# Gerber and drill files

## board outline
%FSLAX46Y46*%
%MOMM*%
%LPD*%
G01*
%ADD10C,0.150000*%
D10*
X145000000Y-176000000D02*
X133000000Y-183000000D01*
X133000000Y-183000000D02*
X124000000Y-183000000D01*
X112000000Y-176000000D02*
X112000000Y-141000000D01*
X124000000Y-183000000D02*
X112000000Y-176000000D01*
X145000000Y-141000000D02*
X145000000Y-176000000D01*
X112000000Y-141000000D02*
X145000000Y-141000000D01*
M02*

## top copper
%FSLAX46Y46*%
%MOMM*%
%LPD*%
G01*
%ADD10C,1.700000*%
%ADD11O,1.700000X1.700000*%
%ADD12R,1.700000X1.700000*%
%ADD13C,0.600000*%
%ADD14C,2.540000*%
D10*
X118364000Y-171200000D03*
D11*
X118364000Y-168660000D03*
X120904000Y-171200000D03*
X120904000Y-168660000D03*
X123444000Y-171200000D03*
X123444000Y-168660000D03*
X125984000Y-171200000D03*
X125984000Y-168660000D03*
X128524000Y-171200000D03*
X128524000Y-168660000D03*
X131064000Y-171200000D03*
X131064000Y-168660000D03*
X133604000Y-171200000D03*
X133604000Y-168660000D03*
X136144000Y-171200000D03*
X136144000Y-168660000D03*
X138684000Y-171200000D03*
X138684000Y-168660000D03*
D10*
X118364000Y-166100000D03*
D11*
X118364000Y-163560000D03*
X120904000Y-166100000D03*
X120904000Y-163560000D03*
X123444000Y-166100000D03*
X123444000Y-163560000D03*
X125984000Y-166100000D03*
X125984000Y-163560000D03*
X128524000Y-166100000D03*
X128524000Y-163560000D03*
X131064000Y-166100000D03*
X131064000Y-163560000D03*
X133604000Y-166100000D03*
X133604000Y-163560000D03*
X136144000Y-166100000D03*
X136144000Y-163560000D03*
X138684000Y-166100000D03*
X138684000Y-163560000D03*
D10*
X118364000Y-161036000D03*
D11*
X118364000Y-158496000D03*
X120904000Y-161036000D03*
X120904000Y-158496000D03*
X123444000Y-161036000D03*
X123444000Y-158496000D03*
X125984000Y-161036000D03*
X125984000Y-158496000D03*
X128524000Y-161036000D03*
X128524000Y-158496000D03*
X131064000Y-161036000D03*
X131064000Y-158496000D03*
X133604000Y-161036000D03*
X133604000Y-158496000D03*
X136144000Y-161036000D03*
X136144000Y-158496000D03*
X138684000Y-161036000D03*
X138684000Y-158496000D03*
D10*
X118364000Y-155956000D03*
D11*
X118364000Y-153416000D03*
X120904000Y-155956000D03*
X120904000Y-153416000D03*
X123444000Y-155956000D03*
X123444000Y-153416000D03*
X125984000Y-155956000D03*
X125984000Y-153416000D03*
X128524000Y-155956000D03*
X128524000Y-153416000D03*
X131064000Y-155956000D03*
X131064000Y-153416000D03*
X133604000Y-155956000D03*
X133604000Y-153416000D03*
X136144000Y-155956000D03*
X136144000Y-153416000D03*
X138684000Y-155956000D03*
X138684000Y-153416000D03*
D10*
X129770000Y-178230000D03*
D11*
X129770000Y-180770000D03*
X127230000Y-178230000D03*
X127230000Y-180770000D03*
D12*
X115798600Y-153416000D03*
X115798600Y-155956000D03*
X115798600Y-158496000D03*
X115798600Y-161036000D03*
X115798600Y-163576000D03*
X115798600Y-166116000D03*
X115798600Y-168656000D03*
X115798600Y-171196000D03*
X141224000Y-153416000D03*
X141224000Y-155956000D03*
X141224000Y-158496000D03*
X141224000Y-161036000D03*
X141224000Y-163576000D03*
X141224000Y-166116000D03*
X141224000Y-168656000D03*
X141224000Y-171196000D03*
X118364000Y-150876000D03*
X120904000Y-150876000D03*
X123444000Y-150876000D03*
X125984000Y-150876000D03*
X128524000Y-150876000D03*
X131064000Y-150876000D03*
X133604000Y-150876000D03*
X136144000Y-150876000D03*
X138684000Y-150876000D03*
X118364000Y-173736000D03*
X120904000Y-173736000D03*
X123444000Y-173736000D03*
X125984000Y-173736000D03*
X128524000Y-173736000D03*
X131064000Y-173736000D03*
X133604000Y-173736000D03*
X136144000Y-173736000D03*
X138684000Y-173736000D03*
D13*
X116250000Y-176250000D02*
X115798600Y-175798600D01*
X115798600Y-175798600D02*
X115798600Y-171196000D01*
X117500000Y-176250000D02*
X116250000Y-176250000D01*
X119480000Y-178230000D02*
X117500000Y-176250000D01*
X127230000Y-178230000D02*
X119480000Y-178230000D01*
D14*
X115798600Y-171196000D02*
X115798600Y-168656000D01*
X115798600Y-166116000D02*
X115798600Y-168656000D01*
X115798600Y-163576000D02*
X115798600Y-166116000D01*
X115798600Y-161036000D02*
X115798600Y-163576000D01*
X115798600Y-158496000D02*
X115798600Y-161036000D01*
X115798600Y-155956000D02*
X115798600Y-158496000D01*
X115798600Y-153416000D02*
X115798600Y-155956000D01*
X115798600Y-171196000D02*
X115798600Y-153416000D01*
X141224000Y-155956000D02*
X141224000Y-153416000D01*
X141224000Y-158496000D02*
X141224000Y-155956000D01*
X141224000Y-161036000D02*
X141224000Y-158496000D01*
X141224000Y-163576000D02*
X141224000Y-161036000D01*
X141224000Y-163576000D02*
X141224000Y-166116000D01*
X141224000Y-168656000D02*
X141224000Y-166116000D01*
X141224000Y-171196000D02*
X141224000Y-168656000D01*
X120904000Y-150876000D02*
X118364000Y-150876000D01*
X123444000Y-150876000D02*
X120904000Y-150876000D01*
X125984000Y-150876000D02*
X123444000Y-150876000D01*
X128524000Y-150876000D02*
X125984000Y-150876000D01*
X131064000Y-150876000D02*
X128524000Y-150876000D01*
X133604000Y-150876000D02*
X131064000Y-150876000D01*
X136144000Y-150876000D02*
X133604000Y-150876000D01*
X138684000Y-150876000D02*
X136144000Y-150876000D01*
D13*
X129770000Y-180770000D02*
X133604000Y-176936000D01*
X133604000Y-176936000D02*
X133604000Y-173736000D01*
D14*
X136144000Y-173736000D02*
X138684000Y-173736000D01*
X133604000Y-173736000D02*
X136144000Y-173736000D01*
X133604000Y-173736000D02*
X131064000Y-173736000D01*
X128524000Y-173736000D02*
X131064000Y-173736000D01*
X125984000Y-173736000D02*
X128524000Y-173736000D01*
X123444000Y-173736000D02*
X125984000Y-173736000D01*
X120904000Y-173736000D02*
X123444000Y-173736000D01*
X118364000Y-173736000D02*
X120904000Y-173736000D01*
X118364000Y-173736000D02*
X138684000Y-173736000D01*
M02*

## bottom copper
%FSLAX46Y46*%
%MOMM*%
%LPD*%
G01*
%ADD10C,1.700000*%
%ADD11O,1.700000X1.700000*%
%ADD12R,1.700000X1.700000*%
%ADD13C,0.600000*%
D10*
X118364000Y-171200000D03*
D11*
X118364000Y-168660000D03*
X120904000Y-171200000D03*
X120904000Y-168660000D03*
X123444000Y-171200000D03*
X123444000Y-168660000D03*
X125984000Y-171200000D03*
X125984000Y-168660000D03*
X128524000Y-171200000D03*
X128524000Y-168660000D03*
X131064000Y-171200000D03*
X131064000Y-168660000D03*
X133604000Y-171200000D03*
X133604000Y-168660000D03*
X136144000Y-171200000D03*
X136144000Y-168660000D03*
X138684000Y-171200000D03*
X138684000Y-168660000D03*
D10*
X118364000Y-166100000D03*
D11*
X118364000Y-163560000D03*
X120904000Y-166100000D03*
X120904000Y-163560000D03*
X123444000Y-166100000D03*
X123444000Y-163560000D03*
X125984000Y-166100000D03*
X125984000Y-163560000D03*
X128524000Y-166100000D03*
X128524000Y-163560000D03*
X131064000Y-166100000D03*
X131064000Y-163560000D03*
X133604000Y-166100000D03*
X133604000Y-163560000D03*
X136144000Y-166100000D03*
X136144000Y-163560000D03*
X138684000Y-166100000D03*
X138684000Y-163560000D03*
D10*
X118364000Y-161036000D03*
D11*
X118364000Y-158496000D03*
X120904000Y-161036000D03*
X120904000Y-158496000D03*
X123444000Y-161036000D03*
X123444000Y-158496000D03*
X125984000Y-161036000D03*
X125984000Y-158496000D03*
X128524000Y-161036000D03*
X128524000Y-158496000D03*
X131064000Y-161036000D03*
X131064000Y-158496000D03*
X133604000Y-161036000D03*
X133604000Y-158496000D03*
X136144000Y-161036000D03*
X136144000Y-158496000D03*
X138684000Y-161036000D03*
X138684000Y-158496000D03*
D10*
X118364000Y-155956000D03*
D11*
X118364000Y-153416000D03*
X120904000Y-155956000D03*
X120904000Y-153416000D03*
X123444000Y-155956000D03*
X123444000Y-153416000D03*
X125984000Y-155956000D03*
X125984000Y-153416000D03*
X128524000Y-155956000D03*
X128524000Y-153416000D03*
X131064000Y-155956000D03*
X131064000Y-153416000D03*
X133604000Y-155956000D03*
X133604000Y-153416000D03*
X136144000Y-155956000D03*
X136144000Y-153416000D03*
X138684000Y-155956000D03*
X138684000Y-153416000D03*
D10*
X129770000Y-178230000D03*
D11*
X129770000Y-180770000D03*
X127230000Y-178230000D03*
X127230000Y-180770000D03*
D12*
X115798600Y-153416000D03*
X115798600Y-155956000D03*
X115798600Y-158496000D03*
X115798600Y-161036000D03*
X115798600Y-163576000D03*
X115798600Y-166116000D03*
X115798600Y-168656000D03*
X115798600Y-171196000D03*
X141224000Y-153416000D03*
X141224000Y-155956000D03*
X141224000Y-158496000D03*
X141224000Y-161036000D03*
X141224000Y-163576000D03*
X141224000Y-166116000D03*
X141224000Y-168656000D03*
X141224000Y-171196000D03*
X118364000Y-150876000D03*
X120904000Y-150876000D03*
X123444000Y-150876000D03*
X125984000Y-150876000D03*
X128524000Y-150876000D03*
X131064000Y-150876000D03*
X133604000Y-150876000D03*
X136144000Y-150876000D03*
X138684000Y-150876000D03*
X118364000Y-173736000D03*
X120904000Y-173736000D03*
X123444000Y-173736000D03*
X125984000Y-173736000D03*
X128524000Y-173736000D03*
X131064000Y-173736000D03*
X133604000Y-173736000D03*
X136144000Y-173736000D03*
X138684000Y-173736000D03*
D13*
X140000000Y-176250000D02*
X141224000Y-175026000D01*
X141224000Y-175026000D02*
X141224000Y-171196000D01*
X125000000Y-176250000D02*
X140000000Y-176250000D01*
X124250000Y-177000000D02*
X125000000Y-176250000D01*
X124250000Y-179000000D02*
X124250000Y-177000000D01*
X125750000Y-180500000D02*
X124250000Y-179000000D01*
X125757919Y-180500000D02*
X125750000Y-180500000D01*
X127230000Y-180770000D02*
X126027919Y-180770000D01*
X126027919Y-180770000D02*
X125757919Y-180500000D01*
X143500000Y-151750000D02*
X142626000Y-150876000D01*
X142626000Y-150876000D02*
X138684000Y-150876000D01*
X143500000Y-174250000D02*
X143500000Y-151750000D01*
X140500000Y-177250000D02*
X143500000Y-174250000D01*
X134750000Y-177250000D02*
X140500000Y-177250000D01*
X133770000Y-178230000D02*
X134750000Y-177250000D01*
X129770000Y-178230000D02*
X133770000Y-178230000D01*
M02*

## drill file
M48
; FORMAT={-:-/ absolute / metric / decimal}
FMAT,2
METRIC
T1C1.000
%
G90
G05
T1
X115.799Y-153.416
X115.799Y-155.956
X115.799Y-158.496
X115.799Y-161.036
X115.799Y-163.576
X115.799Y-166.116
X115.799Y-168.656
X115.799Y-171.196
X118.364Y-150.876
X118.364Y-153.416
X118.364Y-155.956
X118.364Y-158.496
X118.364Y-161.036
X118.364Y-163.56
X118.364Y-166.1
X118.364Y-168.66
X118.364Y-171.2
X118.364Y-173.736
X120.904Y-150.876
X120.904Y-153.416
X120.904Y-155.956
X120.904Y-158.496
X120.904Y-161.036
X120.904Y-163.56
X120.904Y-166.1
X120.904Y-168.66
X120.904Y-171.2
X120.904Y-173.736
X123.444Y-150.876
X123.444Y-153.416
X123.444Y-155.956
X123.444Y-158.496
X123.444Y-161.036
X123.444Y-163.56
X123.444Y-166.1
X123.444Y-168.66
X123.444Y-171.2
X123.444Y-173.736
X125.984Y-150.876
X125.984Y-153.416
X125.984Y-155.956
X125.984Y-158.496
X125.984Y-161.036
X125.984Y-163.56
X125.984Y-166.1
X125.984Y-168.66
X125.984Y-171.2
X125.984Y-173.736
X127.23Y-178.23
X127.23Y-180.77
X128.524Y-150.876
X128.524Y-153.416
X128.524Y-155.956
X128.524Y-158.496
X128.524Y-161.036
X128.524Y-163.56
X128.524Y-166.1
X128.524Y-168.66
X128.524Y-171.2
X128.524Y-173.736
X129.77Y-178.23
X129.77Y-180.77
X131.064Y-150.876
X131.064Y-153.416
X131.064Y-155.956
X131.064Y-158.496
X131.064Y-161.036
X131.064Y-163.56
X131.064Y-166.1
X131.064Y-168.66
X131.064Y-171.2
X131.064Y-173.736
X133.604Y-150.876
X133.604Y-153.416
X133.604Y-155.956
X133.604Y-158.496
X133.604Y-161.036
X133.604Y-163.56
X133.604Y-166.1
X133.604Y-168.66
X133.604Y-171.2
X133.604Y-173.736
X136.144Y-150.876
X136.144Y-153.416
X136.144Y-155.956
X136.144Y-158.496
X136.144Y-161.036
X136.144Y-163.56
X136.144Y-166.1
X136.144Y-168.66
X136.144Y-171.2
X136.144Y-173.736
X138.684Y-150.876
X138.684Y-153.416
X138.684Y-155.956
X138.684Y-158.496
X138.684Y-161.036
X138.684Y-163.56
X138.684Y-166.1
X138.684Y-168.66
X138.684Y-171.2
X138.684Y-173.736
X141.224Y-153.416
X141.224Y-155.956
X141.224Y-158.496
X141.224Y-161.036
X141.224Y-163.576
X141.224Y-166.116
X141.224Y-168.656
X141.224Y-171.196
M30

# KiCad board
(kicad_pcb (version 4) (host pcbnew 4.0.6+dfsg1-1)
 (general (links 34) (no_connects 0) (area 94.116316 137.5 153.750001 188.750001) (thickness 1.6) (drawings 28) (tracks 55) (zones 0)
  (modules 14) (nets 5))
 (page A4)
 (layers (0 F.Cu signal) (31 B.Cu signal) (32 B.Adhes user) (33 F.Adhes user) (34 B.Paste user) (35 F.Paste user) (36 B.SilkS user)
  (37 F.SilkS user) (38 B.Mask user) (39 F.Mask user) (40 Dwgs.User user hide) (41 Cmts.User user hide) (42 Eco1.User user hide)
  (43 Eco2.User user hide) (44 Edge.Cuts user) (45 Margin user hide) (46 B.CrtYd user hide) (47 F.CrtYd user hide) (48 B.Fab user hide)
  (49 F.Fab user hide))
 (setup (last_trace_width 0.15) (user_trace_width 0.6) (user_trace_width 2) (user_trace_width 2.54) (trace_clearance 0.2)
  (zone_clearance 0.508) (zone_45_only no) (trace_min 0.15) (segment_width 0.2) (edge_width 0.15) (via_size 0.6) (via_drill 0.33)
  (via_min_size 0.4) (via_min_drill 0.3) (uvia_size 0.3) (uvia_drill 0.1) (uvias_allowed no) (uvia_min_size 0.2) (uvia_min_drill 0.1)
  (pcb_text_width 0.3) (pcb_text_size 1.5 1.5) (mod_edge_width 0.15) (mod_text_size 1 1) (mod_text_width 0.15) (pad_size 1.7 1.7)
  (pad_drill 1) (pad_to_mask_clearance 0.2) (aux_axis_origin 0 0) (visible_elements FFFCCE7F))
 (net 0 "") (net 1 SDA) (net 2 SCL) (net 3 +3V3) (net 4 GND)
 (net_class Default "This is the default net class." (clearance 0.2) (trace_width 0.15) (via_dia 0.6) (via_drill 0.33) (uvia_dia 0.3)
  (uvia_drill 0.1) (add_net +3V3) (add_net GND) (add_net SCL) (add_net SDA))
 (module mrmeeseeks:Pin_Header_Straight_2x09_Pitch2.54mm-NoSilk (layer F.Cu) (at 118.364 171.2 90)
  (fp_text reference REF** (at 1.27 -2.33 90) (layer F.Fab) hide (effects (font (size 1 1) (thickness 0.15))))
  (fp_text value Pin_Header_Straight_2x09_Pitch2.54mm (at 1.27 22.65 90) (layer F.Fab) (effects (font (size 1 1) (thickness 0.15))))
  (pad 1 thru_hole circle (at 0 0 90) (size 1.7 1.7) (drill 1) (layers *.Cu *.Mask))
  (pad 2 thru_hole oval (at 2.54 0 90) (size 1.7 1.7) (drill 1) (layers *.Cu *.Mask))
  (pad 3 thru_hole oval (at 0 2.54 90) (size 1.7 1.7) (drill 1) (layers *.Cu *.Mask))
  (pad 4 thru_hole oval (at 2.54 2.54 90) (size 1.7 1.7) (drill 1) (layers *.Cu *.Mask))
  (pad 5 thru_hole oval (at 0 5.08 90) (size 1.7 1.7) (drill 1) (layers *.Cu *.Mask))
  (pad 6 thru_hole oval (at 2.54 5.08 90) (size 1.7 1.7) (drill 1) (layers *.Cu *.Mask))
  (pad 7 thru_hole oval (at 0 7.62 90) (size 1.7 1.7) (drill 1) (layers *.Cu *.Mask))
  (pad 8 thru_hole oval (at 2.54 7.62 90) (size 1.7 1.7) (drill 1) (layers *.Cu *.Mask))
  (pad 9 thru_hole oval (at 0 10.16 90) (size 1.7 1.7) (drill 1) (layers *.Cu *.Mask))
  (pad 10 thru_hole oval (at 2.54 10.16 90) (size 1.7 1.7) (drill 1) (layers *.Cu *.Mask))
  (pad 11 thru_hole oval (at 0 12.7 90) (size 1.7 1.7) (drill 1) (layers *.Cu *.Mask))
  (pad 12 thru_hole oval (at 2.54 12.7 90) (size 1.7 1.7) (drill 1) (layers *.Cu *.Mask))
  (pad 13 thru_hole oval (at 0 15.24 90) (size 1.7 1.7) (drill 1) (layers *.Cu *.Mask))
  (pad 14 thru_hole oval (at 2.54 15.24 90) (size 1.7 1.7) (drill 1) (layers *.Cu *.Mask))
  (pad 15 thru_hole oval (at 0 17.78 90) (size 1.7 1.7) (drill 1) (layers *.Cu *.Mask))
  (pad 16 thru_hole oval (at 2.54 17.78 90) (size 1.7 1.7) (drill 1) (layers *.Cu *.Mask))
  (pad 17 thru_hole oval (at 0 20.32 90) (size 1.7 1.7) (drill 1) (layers *.Cu *.Mask))
  (pad 18 thru_hole oval (at 2.54 20.32 90) (size 1.7 1.7) (drill 1) (layers *.Cu *.Mask)))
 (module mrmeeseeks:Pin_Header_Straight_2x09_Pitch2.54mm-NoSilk (layer F.Cu) (at 118.364 166.1 90)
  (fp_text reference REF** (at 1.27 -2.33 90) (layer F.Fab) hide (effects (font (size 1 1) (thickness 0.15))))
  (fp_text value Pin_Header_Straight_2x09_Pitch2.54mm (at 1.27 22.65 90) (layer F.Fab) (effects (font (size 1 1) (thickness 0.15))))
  (pad 1 thru_hole circle (at 0 0 90) (size 1.7 1.7) (drill 1) (layers *.Cu *.Mask))
  (pad 2 thru_hole oval (at 2.54 0 90) (size 1.7 1.7) (drill 1) (layers *.Cu *.Mask))
  (pad 3 thru_hole oval (at 0 2.54 90) (size 1.7 1.7) (drill 1) (layers *.Cu *.Mask))
  (pad 4 thru_hole oval (at 2.54 2.54 90) (size 1.7 1.7) (drill 1) (layers *.Cu *.Mask))
  (pad 5 thru_hole oval (at 0 5.08 90) (size 1.7 1.7) (drill 1) (layers *.Cu *.Mask))
  (pad 6 thru_hole oval (at 2.54 5.08 90) (size 1.7 1.7) (drill 1) (layers *.Cu *.Mask))
  (pad 7 thru_hole oval (at 0 7.62 90) (size 1.7 1.7) (drill 1) (layers *.Cu *.Mask))
  (pad 8 thru_hole oval (at 2.54 7.62 90) (size 1.7 1.7) (drill 1) (layers *.Cu *.Mask))
  (pad 9 thru_hole oval (at 0 10.16 90) (size 1.7 1.7) (drill 1) (layers *.Cu *.Mask))
  (pad 10 thru_hole oval (at 2.54 10.16 90) (size 1.7 1.7) (drill 1) (layers *.Cu *.Mask))
  (pad 11 thru_hole oval (at 0 12.7 90) (size 1.7 1.7) (drill 1) (layers *.Cu *.Mask))
  (pad 12 thru_hole oval (at 2.54 12.7 90) (size 1.7 1.7) (drill 1) (layers *.Cu *.Mask))
  (pad 13 thru_hole oval (at 0 15.24 90) (size 1.7 1.7) (drill 1) (layers *.Cu *.Mask))
  (pad 14 thru_hole oval (at 2.54 15.24 90) (size 1.7 1.7) (drill 1) (layers *.Cu *.Mask))
  (pad 15 thru_hole oval (at 0 17.78 90) (size 1.7 1.7) (drill 1) (layers *.Cu *.Mask))
  (pad 16 thru_hole oval (at 2.54 17.78 90) (size 1.7 1.7) (drill 1) (layers *.Cu *.Mask))
  (pad 17 thru_hole oval (at 0 20.32 90) (size 1.7 1.7) (drill 1) (layers *.Cu *.Mask))
  (pad 18 thru_hole oval (at 2.54 20.32 90) (size 1.7 1.7) (drill 1) (layers *.Cu *.Mask)))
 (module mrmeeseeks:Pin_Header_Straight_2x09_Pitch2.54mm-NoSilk (layer F.Cu) (at 118.364 161.036 90)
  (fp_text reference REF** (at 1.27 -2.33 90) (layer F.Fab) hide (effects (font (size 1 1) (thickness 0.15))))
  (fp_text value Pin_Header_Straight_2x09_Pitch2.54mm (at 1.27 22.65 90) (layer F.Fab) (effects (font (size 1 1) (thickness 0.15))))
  (pad 1 thru_hole circle (at 0 0 90) (size 1.7 1.7) (drill 1) (layers *.Cu *.Mask))
  (pad 2 thru_hole oval (at 2.54 0 90) (size 1.7 1.7) (drill 1) (layers *.Cu *.Mask))
  (pad 3 thru_hole oval (at 0 2.54 90) (size 1.7 1.7) (drill 1) (layers *.Cu *.Mask))
  (pad 4 thru_hole oval (at 2.54 2.54 90) (size 1.7 1.7) (drill 1) (layers *.Cu *.Mask))
  (pad 5 thru_hole oval (at 0 5.08 90) (size 1.7 1.7) (drill 1) (layers *.Cu *.Mask))
  (pad 6 thru_hole oval (at 2.54 5.08 90) (size 1.7 1.7) (drill 1) (layers *.Cu *.Mask))
  (pad 7 thru_hole oval (at 0 7.62 90) (size 1.7 1.7) (drill 1) (layers *.Cu *.Mask))
  (pad 8 thru_hole oval (at 2.54 7.62 90) (size 1.7 1.7) (drill 1) (layers *.Cu *.Mask))
  (pad 9 thru_hole oval (at 0 10.16 90) (size 1.7 1.7) (drill 1) (layers *.Cu *.Mask))
  (pad 10 thru_hole oval (at 2.54 10.16 90) (size 1.7 1.7) (drill 1) (layers *.Cu *.Mask))
  (pad 11 thru_hole oval (at 0 12.7 90) (size 1.7 1.7) (drill 1) (layers *.Cu *.Mask))
  (pad 12 thru_hole oval (at 2.54 12.7 90) (size 1.7 1.7) (drill 1) (layers *.Cu *.Mask))
  (pad 13 thru_hole oval (at 0 15.24 90) (size 1.7 1.7) (drill 1) (layers *.Cu *.Mask))
  (pad 14 thru_hole oval (at 2.54 15.24 90) (size 1.7 1.7) (drill 1) (layers *.Cu *.Mask))
  (pad 15 thru_hole oval (at 0 17.78 90) (size 1.7 1.7) (drill 1) (layers *.Cu *.Mask))
  (pad 16 thru_hole oval (at 2.54 17.78 90) (size 1.7 1.7) (drill 1) (layers *.Cu *.Mask))
  (pad 17 thru_hole oval (at 0 20.32 90) (size 1.7 1.7) (drill 1) (layers *.Cu *.Mask))
  (pad 18 thru_hole oval (at 2.54 20.32 90) (size 1.7 1.7) (drill 1) (layers *.Cu *.Mask)))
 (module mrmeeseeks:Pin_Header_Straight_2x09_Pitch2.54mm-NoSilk (layer F.Cu) (at 118.364 155.956 90)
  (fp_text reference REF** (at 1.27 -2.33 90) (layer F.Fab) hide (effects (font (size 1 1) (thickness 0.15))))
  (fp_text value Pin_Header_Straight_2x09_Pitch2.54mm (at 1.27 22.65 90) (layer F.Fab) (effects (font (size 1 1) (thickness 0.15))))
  (pad 1 thru_hole circle (at 0 0 90) (size 1.7 1.7) (drill 1) (layers *.Cu *.Mask))
  (pad 2 thru_hole oval (at 2.54 0 90) (size 1.7 1.7) (drill 1) (layers *.Cu *.Mask))
  (pad 3 thru_hole oval (at 0 2.54 90) (size 1.7 1.7) (drill 1) (layers *.Cu *.Mask))
  (pad 4 thru_hole oval (at 2.54 2.54 90) (size 1.7 1.7) (drill 1) (layers *.Cu *.Mask))
  (pad 5 thru_hole oval (at 0 5.08 90) (size 1.7 1.7) (drill 1) (layers *.Cu *.Mask))
  (pad 6 thru_hole oval (at 2.54 5.08 90) (size 1.7 1.7) (drill 1) (layers *.Cu *.Mask))
  (pad 7 thru_hole oval (at 0 7.62 90) (size 1.7 1.7) (drill 1) (layers *.Cu *.Mask))
  (pad 8 thru_hole oval (at 2.54 7.62 90) (size 1.7 1.7) (drill 1) (layers *.Cu *.Mask))
  (pad 9 thru_hole oval (at 0 10.16 90) (size 1.7 1.7) (drill 1) (layers *.Cu *.Mask))
  (pad 10 thru_hole oval (at 2.54 10.16 90) (size 1.7 1.7) (drill 1) (layers *.Cu *.Mask))
  (pad 11 thru_hole oval (at 0 12.7 90) (size 1.7 1.7) (drill 1) (layers *.Cu *.Mask))
  (pad 12 thru_hole oval (at 2.54 12.7 90) (size 1.7 1.7) (drill 1) (layers *.Cu *.Mask))
  (pad 13 thru_hole oval (at 0 15.24 90) (size 1.7 1.7) (drill 1) (layers *.Cu *.Mask))
  (pad 14 thru_hole oval (at 2.54 15.24 90) (size 1.7 1.7) (drill 1) (layers *.Cu *.Mask))
  (pad 15 thru_hole oval (at 0 17.78 90) (size 1.7 1.7) (drill 1) (layers *.Cu *.Mask))
  (pad 16 thru_hole oval (at 2.54 17.78 90) (size 1.7 1.7) (drill 1) (layers *.Cu *.Mask))
  (pad 17 thru_hole oval (at 0 20.32 90) (size 1.7 1.7) (drill 1) (layers *.Cu *.Mask))
  (pad 18 thru_hole oval (at 2.54 20.32 90) (size 1.7 1.7) (drill 1) (layers *.Cu *.Mask)))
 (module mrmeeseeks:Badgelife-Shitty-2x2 (layer F.Cu) (at 128.5 179.5)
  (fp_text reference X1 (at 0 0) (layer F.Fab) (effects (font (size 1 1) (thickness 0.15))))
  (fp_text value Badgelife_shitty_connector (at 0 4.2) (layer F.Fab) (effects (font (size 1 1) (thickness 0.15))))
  (pad 4 thru_hole circle (at 1.27 -1.27) (size 1.7 1.7) (drill 1) (layers *.Cu *.Mask) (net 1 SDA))
  (pad 3 thru_hole oval (at 1.27 1.27) (size 1.7 1.7) (drill 1) (layers *.Cu *.Mask) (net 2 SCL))
  (pad 1 thru_hole oval (at -1.27 -1.27) (size 1.7 1.7) (drill 1) (layers *.Cu *.Mask) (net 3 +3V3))
  (pad 2 thru_hole oval (at -1.27 1.27) (size 1.7 1.7) (drill 1) (layers *.Cu *.Mask) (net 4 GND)))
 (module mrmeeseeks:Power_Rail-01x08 (layer F.Cu) (at 115.7986 153.416)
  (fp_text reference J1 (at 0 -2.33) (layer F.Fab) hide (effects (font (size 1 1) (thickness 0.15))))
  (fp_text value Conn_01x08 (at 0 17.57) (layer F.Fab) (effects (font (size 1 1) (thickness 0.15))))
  (pad 1 thru_hole rect (at 0 0) (size 1.7 1.7) (drill 1) (layers *.Cu *.Mask) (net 3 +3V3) (solder_mask_margin 0.1))
  (pad 2 thru_hole rect (at 0 2.54) (size 1.7 1.7) (drill 1) (layers *.Cu *.Mask) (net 3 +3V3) (solder_mask_margin 0.1))
  (pad 3 thru_hole rect (at 0 5.08) (size 1.7 1.7) (drill 1) (layers *.Cu *.Mask) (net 3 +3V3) (solder_mask_margin 0.1))
  (pad 4 thru_hole rect (at 0 7.62) (size 1.7 1.7) (drill 1) (layers *.Cu *.Mask) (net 3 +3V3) (solder_mask_margin 0.1))
  (pad 5 thru_hole rect (at 0 10.16) (size 1.7 1.7) (drill 1) (layers *.Cu *.Mask) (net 3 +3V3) (solder_mask_margin 0.1))
  (pad 6 thru_hole rect (at 0 12.7) (size 1.7 1.7) (drill 1) (layers *.Cu *.Mask) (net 3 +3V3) (solder_mask_margin 0.1))
  (pad 7 thru_hole rect (at 0 15.24) (size 1.7 1.7) (drill 1) (layers *.Cu *.Mask) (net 3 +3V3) (solder_mask_margin 0.1))
  (pad 8 thru_hole rect (at 0 17.78) (size 1.7 1.7) (drill 1) (layers *.Cu *.Mask) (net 3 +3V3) (solder_mask_margin 0.1)))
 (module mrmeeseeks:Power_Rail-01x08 (layer F.Cu) (at 141.224 153.416)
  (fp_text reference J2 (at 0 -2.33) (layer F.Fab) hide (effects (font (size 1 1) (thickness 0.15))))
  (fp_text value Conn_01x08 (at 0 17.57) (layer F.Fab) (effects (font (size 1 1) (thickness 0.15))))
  (pad 1 thru_hole rect (at 0 0) (size 1.7 1.7) (drill 1) (layers *.Cu *.Mask) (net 4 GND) (solder_mask_margin 0.1))
  (pad 2 thru_hole rect (at 0 2.54) (size 1.7 1.7) (drill 1) (layers *.Cu *.Mask) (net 4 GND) (solder_mask_margin 0.1))
  (pad 3 thru_hole rect (at 0 5.08) (size 1.7 1.7) (drill 1) (layers *.Cu *.Mask) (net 4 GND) (solder_mask_margin 0.1))
  (pad 4 thru_hole rect (at 0 7.62) (size 1.7 1.7) (drill 1) (layers *.Cu *.Mask) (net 4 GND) (solder_mask_margin 0.1))
  (pad 5 thru_hole rect (at 0 10.16) (size 1.7 1.7) (drill 1) (layers *.Cu *.Mask) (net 4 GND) (solder_mask_margin 0.1))
  (pad 6 thru_hole rect (at 0 12.7) (size 1.7 1.7) (drill 1) (layers *.Cu *.Mask) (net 4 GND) (solder_mask_margin 0.1))
  (pad 7 thru_hole rect (at 0 15.24) (size 1.7 1.7) (drill 1) (layers *.Cu *.Mask) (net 4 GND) (solder_mask_margin 0.1))
  (pad 8 thru_hole rect (at 0 17.78) (size 1.7 1.7) (drill 1) (layers *.Cu *.Mask) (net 4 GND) (solder_mask_margin 0.1)))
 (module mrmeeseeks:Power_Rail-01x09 (layer F.Cu) (at 118.364 150.876 90)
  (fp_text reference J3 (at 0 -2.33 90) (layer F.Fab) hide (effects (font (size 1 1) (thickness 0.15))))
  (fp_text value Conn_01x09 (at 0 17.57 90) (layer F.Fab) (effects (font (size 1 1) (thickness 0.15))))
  (pad 1 thru_hole rect (at 0 0 90) (size 1.7 1.7) (drill 1) (layers *.Cu *.Mask) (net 1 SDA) (solder_mask_margin 0.1))
  (pad 2 thru_hole rect (at 0 2.54 90) (size 1.7 1.7) (drill 1) (layers *.Cu *.Mask) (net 1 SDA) (solder_mask_margin 0.1))
  (pad 3 thru_hole rect (at 0 5.08 90) (size 1.7 1.7) (drill 1) (layers *.Cu *.Mask) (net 1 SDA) (solder_mask_margin 0.1))
  (pad 4 thru_hole rect (at 0 7.62 90) (size 1.7 1.7) (drill 1) (layers *.Cu *.Mask) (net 1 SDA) (solder_mask_margin 0.1))
  (pad 5 thru_hole rect (at 0 10.16 90) (size 1.7 1.7) (drill 1) (layers *.Cu *.Mask) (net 1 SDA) (solder_mask_margin 0.1))
  (pad 6 thru_hole rect (at 0 12.7 90) (size 1.7 1.7) (drill 1) (layers *.Cu *.Mask) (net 1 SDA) (solder_mask_margin 0.1))
  (pad 7 thru_hole rect (at 0 15.24 90) (size 1.7 1.7) (drill 1) (layers *.Cu *.Mask) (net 1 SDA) (solder_mask_margin 0.1))
  (pad 8 thru_hole rect (at 0 17.78 90) (size 1.7 1.7) (drill 1) (layers *.Cu *.Mask) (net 1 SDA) (solder_mask_margin 0.1))
  (pad 9 thru_hole rect (at 0 20.32 90) (size 1.7 1.7) (drill 1) (layers *.Cu *.Mask) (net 1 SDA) (solder_mask_margin 0.1)))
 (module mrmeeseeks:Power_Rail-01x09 (layer F.Cu) (at 118.364 173.736 90)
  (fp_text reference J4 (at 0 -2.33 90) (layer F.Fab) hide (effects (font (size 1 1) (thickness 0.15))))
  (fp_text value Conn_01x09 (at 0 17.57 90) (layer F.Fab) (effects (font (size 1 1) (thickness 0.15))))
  (pad 1 thru_hole rect (at 0 0 90) (size 1.7 1.7) (drill 1) (layers *.Cu *.Mask) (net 2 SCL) (solder_mask_margin 0.1))
  (pad 2 thru_hole rect (at 0 2.54 90) (size 1.7 1.7) (drill 1) (layers *.Cu *.Mask) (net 2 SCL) (solder_mask_margin 0.1))
  (pad 3 thru_hole rect (at 0 5.08 90) (size 1.7 1.7) (drill 1) (layers *.Cu *.Mask) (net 2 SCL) (solder_mask_margin 0.1))
  (pad 4 thru_hole rect (at 0 7.62 90) (size 1.7 1.7) (drill 1) (layers *.Cu *.Mask) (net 2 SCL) (solder_mask_margin 0.1))
  (pad 5 thru_hole rect (at 0 10.16 90) (size 1.7 1.7) (drill 1) (layers *.Cu *.Mask) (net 2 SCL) (solder_mask_margin 0.1))
  (pad 6 thru_hole rect (at 0 12.7 90) (size 1.7 1.7) (drill 1) (layers *.Cu *.Mask) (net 2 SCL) (solder_mask_margin 0.1))
  (pad 7 thru_hole rect (at 0 15.24 90) (size 1.7 1.7) (drill 1) (layers *.Cu *.Mask) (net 2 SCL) (solder_mask_margin 0.1))
  (pad 8 thru_hole rect (at 0 17.78 90) (size 1.7 1.7) (drill 1) (layers *.Cu *.Mask) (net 2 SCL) (solder_mask_margin 0.1))
  (pad 9 thru_hole rect (at 0 20.32 90) (size 1.7 1.7) (drill 1) (layers *.Cu *.Mask) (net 2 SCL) (solder_mask_margin 0.1)))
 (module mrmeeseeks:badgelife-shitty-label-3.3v (layer F.Cu) (at 113.4 162.2 90)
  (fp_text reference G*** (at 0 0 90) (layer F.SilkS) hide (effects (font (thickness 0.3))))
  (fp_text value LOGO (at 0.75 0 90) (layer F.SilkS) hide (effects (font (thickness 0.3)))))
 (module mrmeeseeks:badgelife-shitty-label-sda (layer F.Cu) (at 128.2 148.8)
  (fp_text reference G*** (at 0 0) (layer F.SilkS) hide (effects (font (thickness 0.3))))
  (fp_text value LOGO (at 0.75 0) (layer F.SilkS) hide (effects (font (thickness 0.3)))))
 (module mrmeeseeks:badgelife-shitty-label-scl (layer F.Cu) (at 128.4 175.7)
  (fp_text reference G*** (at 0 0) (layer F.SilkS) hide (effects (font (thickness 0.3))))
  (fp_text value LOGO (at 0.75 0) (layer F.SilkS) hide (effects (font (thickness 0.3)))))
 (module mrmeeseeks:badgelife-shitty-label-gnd (layer F.Cu) (at 143.7 162.3 270)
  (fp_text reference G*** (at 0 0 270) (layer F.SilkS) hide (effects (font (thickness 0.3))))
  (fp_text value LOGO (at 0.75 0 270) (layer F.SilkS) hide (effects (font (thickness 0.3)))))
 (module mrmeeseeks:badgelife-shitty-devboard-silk (layer F.Cu) (at 128.9 144.6)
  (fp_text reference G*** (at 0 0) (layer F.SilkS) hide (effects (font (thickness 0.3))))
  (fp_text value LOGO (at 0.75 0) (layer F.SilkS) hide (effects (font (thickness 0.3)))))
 (gr_line (start 145 176) (end 133 183) (layer Edge.Cuts) (width 0.15))
 (gr_line (start 133 183) (end 124 183) (layer Edge.Cuts) (width 0.15))
 (gr_line (start 112 176) (end 112 141) (layer Edge.Cuts) (width 0.15))
 (gr_line (start 124 183) (end 112 176) (layer Edge.Cuts) (width 0.15))
 (gr_line (start 145 141) (end 145 176) (layer Edge.Cuts) (width 0.15))
 (gr_line (start 112 141) (end 145 141) (layer Edge.Cuts) (width 0.15))
 (segment (start 116.25 176.25) (end 115.7986 175.7986) (width 0.6) (layer F.Cu) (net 3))
 (segment (start 115.7986 175.7986) (end 115.7986 171.196) (width 0.6) (layer F.Cu) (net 3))
 (segment (start 117.5 176.25) (end 116.25 176.25) (width 0.6) (layer F.Cu) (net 3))
 (segment (start 119.48 178.23) (end 117.5 176.25) (width 0.6) (layer F.Cu) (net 3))
 (segment (start 127.23 178.23) (end 119.48 178.23) (width 0.6) (layer F.Cu) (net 3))
 (segment (start 115.7986 171.196) (end 115.7986 168.656) (width 2.54) (layer F.Cu) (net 3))
 (segment (start 115.7986 166.116) (end 115.7986 168.656) (width 2.54) (layer F.Cu) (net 3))
 (segment (start 115.7986 163.576) (end 115.7986 166.116) (width 2.54) (layer F.Cu) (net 3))
 (segment (start 115.7986 161.036) (end 115.7986 163.576) (width 2.54) (layer F.Cu) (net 3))
 (segment (start 115.7986 158.496) (end 115.7986 161.036) (width 2.54) (layer F.Cu) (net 3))
 (segment (start 115.7986 155.956) (end 115.7986 158.496) (width 2.54) (layer F.Cu) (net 3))
 (segment (start 115.7986 153.416) (end 115.7986 155.956) (width 2.54) (layer F.Cu) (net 3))
 (segment (start 115.7986 171.196) (end 115.7986 153.416) (width 2.54) (layer F.Cu) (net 3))
 (segment (start 140 176.25) (end 141.224 175.026) (width 0.6) (layer B.Cu) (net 4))
 (segment (start 141.224 175.026) (end 141.224 171.196) (width 0.6) (layer B.Cu) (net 4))
 (segment (start 125 176.25) (end 140 176.25) (width 0.6) (layer B.Cu) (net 4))
 (segment (start 124.25 177) (end 125 176.25) (width 0.6) (layer B.Cu) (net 4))
 (segment (start 124.25 179) (end 124.25 177) (width 0.6) (layer B.Cu) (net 4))
 (segment (start 125.75 180.5) (end 124.25 179) (width 0.6) (layer B.Cu) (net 4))
 (segment (start 125.757919 180.5) (end 125.75 180.5) (width 0.6) (layer B.Cu) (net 4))
 (segment (start 127.23 180.77) (end 126.027919 180.77) (width 0.6) (layer B.Cu) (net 4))
 (segment (start 126.027919 180.77) (end 125.757919 180.5) (width 0.6) (layer B.Cu) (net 4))
 (segment (start 141.224 155.956) (end 141.224 153.416) (width 2.54) (layer F.Cu) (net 4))
 (segment (start 141.224 158.496) (end 141.224 155.956) (width 2.54) (layer F.Cu) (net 4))
 (segment (start 141.224 161.036) (end 141.224 158.496) (width 2.54) (layer F.Cu) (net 4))
 (segment (start 141.224 163.576) (end 141.224 161.036) (width 2.54) (layer F.Cu) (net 4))
 (segment (start 141.224 163.576) (end 141.224 166.116) (width 2.54) (layer F.Cu) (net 4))
 (segment (start 141.224 168.656) (end 141.224 166.116) (width 2.54) (layer F.Cu) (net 4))
 (segment (start 141.224 171.196) (end 141.224 168.656) (width 2.54) (layer F.Cu) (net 4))
 (segment (start 143.5 151.75) (end 142.626 150.876) (width 0.6) (layer B.Cu) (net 1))
 (segment (start 142.626 150.876) (end 138.684 150.876) (width 0.6) (layer B.Cu) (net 1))
 (segment (start 143.5 174.25) (end 143.5 151.75) (width 0.6) (layer B.Cu) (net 1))
 (segment (start 140.5 177.25) (end 143.5 174.25) (width 0.6) (layer B.Cu) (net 1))
 (segment (start 134.75 177.25) (end 140.5 177.25) (width 0.6) (layer B.Cu) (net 1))
 (segment (start 133.77 178.23) (end 134.75 177.25) (width 0.6) (layer B.Cu) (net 1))
 (segment (start 129.77 178.23) (end 133.77 178.23) (width 0.6) (layer B.Cu) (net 1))
 (segment (start 120.904 150.876) (end 118.364 150.876) (width 2.54) (layer F.Cu) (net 1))
 (segment (start 123.444 150.876) (end 120.904 150.876) (width 2.54) (layer F.Cu) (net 1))
 (segment (start 125.984 150.876) (end 123.444 150.876) (width 2.54) (layer F.Cu) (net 1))
 (segment (start 128.524 150.876) (end 125.984 150.876) (width 2.54) (layer F.Cu) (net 1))
 (segment (start 131.064 150.876) (end 128.524 150.876) (width 2.54) (layer F.Cu) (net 1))
 (segment (start 133.604 150.876) (end 131.064 150.876) (width 2.54) (layer F.Cu) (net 1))
 (segment (start 136.144 150.876) (end 133.604 150.876) (width 2.54) (layer F.Cu) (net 1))
 (segment (start 138.684 150.876) (end 136.144 150.876) (width 2.54) (layer F.Cu) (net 1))
 (segment (start 129.77 180.77) (end 133.604 176.936) (width 0.6) (layer F.Cu) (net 2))
 (segment (start 133.604 176.936) (end 133.604 173.736) (width 0.6) (layer F.Cu) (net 2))
 (segment (start 136.144 173.736) (end 138.684 173.736) (width 2.54) (layer F.Cu) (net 2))
 (segment (start 133.604 173.736) (end 136.144 173.736) (width 2.54) (layer F.Cu) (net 2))
 (segment (start 133.604 173.736) (end 131.064 173.736) (width 2.54) (layer F.Cu) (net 2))
 (segment (start 128.524 173.736) (end 131.064 173.736) (width 2.54) (layer F.Cu) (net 2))
 (segment (start 125.984 173.736) (end 128.524 173.736) (width 2.54) (layer F.Cu) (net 2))
 (segment (start 123.444 173.736) (end 125.984 173.736) (width 2.54) (layer F.Cu) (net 2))
 (segment (start 120.904 173.736) (end 123.444 173.736) (width 2.54) (layer F.Cu) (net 2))
 (segment (start 118.364 173.736) (end 120.904 173.736) (width 2.54) (layer F.Cu) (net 2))
 (segment (start 118.364 173.736) (end 138.684 173.736) (width 2.54) (layer F.Cu) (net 2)))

